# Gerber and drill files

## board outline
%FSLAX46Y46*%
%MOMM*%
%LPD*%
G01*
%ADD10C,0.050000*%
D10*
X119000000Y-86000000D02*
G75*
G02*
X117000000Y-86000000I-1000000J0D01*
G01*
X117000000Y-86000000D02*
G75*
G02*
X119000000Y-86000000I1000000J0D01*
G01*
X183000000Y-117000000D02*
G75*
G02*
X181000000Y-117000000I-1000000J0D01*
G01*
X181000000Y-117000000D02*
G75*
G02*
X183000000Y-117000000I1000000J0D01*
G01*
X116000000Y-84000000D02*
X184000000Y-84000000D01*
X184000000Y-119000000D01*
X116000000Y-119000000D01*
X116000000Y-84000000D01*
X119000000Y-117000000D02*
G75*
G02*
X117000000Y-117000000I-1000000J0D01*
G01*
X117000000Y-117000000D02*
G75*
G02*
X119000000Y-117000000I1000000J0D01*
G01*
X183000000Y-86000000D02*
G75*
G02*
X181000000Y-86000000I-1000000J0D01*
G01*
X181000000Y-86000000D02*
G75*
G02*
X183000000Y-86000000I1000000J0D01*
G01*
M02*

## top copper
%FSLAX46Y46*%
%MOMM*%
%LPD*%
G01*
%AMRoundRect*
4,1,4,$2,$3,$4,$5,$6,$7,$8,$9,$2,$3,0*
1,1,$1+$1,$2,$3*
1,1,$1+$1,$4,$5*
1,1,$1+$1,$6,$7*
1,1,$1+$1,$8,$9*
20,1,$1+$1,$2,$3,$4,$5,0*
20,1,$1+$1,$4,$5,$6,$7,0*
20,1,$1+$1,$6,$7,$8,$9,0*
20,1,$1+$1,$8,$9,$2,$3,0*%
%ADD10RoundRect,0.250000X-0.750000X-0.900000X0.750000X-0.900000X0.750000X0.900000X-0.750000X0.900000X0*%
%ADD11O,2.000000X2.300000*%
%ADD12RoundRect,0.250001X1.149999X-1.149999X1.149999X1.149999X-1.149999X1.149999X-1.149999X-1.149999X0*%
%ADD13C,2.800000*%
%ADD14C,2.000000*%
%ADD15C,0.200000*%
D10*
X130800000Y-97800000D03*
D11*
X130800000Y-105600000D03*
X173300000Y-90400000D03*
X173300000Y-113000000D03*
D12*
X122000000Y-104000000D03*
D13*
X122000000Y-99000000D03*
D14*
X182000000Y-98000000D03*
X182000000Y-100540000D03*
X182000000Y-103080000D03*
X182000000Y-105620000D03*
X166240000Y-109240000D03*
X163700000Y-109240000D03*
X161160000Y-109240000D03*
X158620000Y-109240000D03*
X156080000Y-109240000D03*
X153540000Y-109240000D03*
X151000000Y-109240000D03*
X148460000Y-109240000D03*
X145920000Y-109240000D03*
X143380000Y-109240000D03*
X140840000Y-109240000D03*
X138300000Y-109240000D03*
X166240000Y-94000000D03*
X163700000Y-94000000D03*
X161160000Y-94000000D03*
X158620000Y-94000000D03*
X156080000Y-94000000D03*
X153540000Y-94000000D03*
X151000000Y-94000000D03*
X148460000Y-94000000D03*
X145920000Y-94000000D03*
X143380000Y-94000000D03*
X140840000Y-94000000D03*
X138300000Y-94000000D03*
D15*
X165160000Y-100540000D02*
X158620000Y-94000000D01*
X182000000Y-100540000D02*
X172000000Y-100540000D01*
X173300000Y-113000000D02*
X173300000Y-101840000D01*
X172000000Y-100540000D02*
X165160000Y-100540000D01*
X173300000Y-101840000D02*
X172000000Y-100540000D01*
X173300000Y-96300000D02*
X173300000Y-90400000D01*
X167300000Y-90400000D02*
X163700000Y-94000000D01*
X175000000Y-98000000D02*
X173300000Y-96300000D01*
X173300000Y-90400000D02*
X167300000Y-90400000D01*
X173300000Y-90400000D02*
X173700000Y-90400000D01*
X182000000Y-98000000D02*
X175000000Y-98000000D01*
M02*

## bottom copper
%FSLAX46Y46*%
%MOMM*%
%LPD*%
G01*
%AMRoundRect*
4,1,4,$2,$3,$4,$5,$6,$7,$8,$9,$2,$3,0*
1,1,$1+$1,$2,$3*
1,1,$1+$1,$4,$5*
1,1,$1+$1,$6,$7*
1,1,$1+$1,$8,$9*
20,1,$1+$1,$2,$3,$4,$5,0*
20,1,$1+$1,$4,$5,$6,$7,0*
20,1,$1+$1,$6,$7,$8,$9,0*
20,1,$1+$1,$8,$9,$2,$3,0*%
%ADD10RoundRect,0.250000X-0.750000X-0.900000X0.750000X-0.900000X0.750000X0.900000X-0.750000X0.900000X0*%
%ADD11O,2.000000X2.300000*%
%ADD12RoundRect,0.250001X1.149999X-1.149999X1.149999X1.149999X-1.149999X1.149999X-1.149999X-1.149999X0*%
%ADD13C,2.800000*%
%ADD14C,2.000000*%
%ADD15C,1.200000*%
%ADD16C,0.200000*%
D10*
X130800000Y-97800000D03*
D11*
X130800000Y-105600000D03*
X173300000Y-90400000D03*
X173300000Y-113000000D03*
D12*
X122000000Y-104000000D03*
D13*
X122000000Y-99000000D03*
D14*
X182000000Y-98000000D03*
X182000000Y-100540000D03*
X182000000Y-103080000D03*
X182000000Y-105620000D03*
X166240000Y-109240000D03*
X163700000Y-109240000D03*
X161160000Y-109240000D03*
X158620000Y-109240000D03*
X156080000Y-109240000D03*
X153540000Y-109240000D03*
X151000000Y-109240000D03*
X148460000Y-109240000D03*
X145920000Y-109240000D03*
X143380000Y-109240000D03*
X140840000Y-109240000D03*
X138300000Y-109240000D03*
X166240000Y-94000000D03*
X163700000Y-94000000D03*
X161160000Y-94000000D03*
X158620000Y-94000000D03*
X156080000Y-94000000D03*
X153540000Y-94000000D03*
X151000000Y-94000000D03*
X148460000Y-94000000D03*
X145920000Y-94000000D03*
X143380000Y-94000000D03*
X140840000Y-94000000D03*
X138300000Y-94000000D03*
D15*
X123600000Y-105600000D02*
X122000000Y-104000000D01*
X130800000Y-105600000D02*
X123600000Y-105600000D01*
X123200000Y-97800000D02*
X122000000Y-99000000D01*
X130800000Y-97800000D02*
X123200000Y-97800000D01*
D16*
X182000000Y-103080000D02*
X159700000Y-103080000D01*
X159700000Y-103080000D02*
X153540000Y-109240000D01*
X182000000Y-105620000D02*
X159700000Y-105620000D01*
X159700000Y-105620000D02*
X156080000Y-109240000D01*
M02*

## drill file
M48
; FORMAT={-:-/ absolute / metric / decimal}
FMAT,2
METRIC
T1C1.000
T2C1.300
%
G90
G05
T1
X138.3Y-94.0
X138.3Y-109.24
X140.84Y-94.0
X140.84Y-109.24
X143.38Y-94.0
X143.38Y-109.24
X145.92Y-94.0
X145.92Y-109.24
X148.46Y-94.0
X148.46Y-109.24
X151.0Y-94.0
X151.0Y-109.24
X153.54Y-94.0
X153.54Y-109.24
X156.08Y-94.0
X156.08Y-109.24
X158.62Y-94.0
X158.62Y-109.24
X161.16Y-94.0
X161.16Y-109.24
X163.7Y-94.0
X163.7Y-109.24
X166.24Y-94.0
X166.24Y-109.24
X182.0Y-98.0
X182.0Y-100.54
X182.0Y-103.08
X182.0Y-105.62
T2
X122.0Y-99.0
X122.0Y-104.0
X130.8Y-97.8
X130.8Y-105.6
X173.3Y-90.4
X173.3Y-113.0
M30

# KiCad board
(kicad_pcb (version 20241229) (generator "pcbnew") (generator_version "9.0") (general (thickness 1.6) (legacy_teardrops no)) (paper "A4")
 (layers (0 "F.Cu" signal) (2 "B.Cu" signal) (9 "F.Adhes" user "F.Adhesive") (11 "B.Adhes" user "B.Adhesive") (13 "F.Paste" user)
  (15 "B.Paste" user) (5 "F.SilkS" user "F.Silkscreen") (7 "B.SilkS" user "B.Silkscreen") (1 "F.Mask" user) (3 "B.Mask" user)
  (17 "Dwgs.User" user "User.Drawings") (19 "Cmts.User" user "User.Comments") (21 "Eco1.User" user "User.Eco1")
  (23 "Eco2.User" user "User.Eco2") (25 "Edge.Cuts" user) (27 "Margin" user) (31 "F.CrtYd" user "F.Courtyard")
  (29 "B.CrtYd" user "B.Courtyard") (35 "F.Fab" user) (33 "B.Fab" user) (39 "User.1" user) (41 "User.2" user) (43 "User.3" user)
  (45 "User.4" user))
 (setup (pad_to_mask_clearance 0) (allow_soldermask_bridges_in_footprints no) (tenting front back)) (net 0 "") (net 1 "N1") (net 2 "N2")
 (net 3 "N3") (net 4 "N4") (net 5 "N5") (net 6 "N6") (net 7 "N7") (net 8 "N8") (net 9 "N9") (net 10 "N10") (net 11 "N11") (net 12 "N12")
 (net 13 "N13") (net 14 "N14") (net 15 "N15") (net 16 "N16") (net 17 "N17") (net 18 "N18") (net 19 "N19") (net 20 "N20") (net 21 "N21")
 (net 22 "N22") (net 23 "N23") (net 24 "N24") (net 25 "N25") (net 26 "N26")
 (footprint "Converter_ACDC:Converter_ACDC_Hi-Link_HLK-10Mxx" (layer "F.Cu") (at 130.8 97.8)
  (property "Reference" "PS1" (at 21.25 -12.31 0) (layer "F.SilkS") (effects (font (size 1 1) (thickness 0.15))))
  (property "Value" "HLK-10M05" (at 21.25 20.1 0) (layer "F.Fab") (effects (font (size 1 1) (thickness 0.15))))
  (pad "1" thru_hole roundrect (at 0 0) (size 2 2.3) (drill 1.3) (layers "*.Cu" "*.Mask") (remove_unused_layers no) (roundrect_rratio 0.125)
   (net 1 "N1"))
  (pad "2" thru_hole oval (at 0 7.8) (size 2 2.3) (drill 1.3) (layers "*.Cu" "*.Mask") (remove_unused_layers no) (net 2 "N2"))
  (pad "3" thru_hole oval (at 42.5 -7.4) (size 2 2.3) (drill 1.3) (layers "*.Cu" "*.Mask") (remove_unused_layers no) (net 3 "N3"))
  (pad "4" thru_hole oval (at 42.5 15.2) (size 2 2.3) (drill 1.3) (layers "*.Cu" "*.Mask") (remove_unused_layers no) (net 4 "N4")))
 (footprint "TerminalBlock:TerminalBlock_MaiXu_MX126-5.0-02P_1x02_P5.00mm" (layer "F.Cu") (at 122 104 90)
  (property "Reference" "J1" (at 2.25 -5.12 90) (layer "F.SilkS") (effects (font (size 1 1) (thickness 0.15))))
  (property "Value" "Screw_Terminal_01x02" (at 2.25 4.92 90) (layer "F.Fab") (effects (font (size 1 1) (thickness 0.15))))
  (pad "1" thru_hole roundrect (at 0 0 90) (size 2.8 2.8) (drill 1.3) (layers "*.Cu" "*.Mask") (remove_unused_layers no)
   (roundrect_rratio 0.089286) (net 2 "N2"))
  (pad "2" thru_hole circle (at 5 0 90) (size 2.8 2.8) (drill 1.3) (layers "*.Cu" "*.Mask") (remove_unused_layers no) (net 1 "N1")))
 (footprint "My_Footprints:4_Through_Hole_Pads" (layer "F.Cu") (at 174.38 103.08 -90)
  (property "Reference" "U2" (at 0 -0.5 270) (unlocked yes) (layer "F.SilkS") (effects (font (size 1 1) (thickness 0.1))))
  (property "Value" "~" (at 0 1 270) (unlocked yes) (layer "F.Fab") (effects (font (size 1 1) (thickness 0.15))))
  (pad "1" thru_hole circle (at -5.08 -7.62 270) (size 2 2) (drill 1) (layers "*.Cu" "*.Mask") (remove_unused_layers no) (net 3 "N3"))
  (pad "2" thru_hole circle (at -2.54 -7.62 270) (size 2 2) (drill 1) (layers "*.Cu" "*.Mask") (remove_unused_layers no) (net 4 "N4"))
  (pad "3" thru_hole circle (at 0 -7.62 270) (size 2 2) (drill 1) (layers "*.Cu" "*.Mask") (remove_unused_layers no) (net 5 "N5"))
  (pad "4" thru_hole circle (at 2.54 -7.62 270) (size 2 2) (drill 1) (layers "*.Cu" "*.Mask") (remove_unused_layers no) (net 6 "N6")))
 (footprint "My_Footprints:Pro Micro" (layer "B.Cu") (at 135.76 101.62 90)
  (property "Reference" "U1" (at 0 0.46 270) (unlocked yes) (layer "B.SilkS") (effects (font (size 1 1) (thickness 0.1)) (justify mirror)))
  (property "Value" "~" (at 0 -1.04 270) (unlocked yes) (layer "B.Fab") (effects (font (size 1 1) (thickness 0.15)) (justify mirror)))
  (pad "1" thru_hole circle (at -7.62 30.48 90) (size 2 2) (drill 1) (layers "*.Cu" "*.Mask") (remove_unused_layers no) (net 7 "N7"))
  (pad "2" thru_hole circle (at -7.62 27.94 90) (size 2 2) (drill 1) (layers "*.Cu" "*.Mask") (remove_unused_layers no) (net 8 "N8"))
  (pad "3" thru_hole circle (at -7.62 25.4 90) (size 2 2) (drill 1) (layers "*.Cu" "*.Mask") (remove_unused_layers no) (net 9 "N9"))
  (pad "4" thru_hole circle (at -7.62 22.86 90) (size 2 2) (drill 1) (layers "*.Cu" "*.Mask") (remove_unused_layers no) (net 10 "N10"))
  (pad "5" thru_hole circle (at -7.62 20.32 90) (size 2 2) (drill 1) (layers "*.Cu" "*.Mask") (remove_unused_layers no) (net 6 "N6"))
  (pad "6" thru_hole circle (at -7.62 17.78 90) (size 2 2) (drill 1) (layers "*.Cu" "*.Mask") (remove_unused_layers no) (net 5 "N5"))
  (pad "7" thru_hole circle (at -7.62 15.24 90) (size 2 2) (drill 1) (layers "*.Cu" "*.Mask") (remove_unused_layers no) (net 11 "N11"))
  (pad "8" thru_hole circle (at -7.62 12.7 90) (size 2 2) (drill 1) (layers "*.Cu" "*.Mask") (remove_unused_layers no) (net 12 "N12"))
  (pad "9" thru_hole circle (at -7.62 10.16 90) (size 2 2) (drill 1) (layers "*.Cu" "*.Mask") (remove_unused_layers no) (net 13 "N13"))
  (pad "10" thru_hole circle (at -7.62 7.62 180) (size 2 2) (drill 1) (layers "*.Cu" "*.Mask") (remove_unused_layers no) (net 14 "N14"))
  (pad "11" thru_hole circle (at -7.62 5.08 90) (size 2 2) (drill 1) (layers "*.Cu" "*.Mask") (remove_unused_layers no) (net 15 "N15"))
  (pad "12" thru_hole circle (at -7.62 2.54 90) (size 2 2) (drill 1) (layers "*.Cu" "*.Mask") (remove_unused_layers no) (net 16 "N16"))
  (pad "13" thru_hole circle (at 7.62 30.48 90) (size 2 2) (drill 1) (layers "*.Cu" "*.Mask") (remove_unused_layers no) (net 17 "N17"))
  (pad "14" thru_hole circle (at 7.62 27.94 90) (size 2 2) (drill 1) (layers "*.Cu" "*.Mask") (remove_unused_layers no) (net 3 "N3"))
  (pad "15" thru_hole circle (at 7.62 25.4 270) (size 2 2) (drill 1) (layers "*.Cu" "*.Mask") (remove_unused_layers no) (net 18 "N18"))
  (pad "16" thru_hole circle (at 7.62 22.86) (size 2 2) (drill 1) (layers "*.Cu" "*.Mask") (remove_unused_layers no) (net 4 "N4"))
  (pad "17" thru_hole circle (at 7.62 20.32 90) (size 2 2) (drill 1) (layers "*.Cu" "*.Mask") (remove_unused_layers no) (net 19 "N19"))
  (pad "18" thru_hole circle (at 7.62 17.78 90) (size 2 2) (drill 1) (layers "*.Cu" "*.Mask") (remove_unused_layers no) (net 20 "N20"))
  (pad "19" thru_hole circle (at 7.62 15.24 90) (size 2 2) (drill 1) (layers "*.Cu" "*.Mask") (remove_unused_layers no) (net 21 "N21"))
  (pad "20" thru_hole circle (at 7.62 12.7 90) (size 2 2) (drill 1) (layers "*.Cu" "*.Mask") (remove_unused_layers no) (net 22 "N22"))
  (pad "21" thru_hole circle (at 7.62 10.16 90) (size 2 2) (drill 1) (layers "*.Cu" "*.Mask") (remove_unused_layers no) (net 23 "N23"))
  (pad "22" thru_hole circle (at 7.62 7.62 90) (size 2 2) (drill 1) (layers "*.Cu" "*.Mask") (remove_unused_layers no) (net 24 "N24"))
  (pad "23" thru_hole circle (at 7.62 5.08 90) (size 2 2) (drill 1) (layers "*.Cu" "*.Mask") (remove_unused_layers no) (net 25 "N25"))
  (pad "24" thru_hole circle (at 7.62 2.54 90) (size 2 2) (drill 1) (layers "*.Cu" "*.Mask") (remove_unused_layers no) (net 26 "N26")))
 (gr_circle (center 118 86) (end 119 86) (stroke (width 0.05) (type default)) (fill no) (layer "Edge.Cuts"))
 (gr_circle (center 182 117) (end 182 118) (stroke (width 0.05) (type default)) (fill no) (layer "Edge.Cuts"))
 (gr_rect (start 116 84) (end 184 119) (stroke (width 0.05) (type default)) (fill no) (layer "Edge.Cuts"))
 (gr_circle (center 118 117) (end 119 117) (stroke (width 0.05) (type default)) (fill no) (layer "Edge.Cuts"))
 (gr_circle (center 182 86) (end 183 86) (stroke (width 0.05) (type default)) (fill no) (layer "Edge.Cuts"))
 (segment (start 123.6 105.6) (end 122 104) (width 1.2) (layer "B.Cu") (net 2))
 (segment (start 130.8 105.6) (end 123.6 105.6) (width 1.2) (layer "B.Cu") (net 2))
 (segment (start 123.2 97.8) (end 122 99) (width 1.2) (layer "B.Cu") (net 1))
 (segment (start 130.8 97.8) (end 123.2 97.8) (width 1.2) (layer "B.Cu") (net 1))
 (segment (start 165.16 100.54) (end 158.62 94) (width 0.2) (layer "F.Cu") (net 4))
 (segment (start 182 100.54) (end 172 100.54) (width 0.2) (layer "F.Cu") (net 4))
 (segment (start 173.3 113) (end 173.3 101.84) (width 0.2) (layer "F.Cu") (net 4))
 (segment (start 172 100.54) (end 165.16 100.54) (width 0.2) (layer "F.Cu") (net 4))
 (segment (start 173.3 101.84) (end 172 100.54) (width 0.2) (layer "F.Cu") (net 4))
 (segment (start 173.3 96.3) (end 173.3 90.4) (width 0.2) (layer "F.Cu") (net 3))
 (segment (start 167.3 90.4) (end 163.7 94) (width 0.2) (layer "F.Cu") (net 3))
 (segment (start 175 98) (end 173.3 96.3) (width 0.2) (layer "F.Cu") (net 3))
 (segment (start 173.3 90.4) (end 167.3 90.4) (width 0.2) (layer "F.Cu") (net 3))
 (segment (start 173.3 90.4) (end 173.7 90.4) (width 0.2) (layer "F.Cu") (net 3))
 (segment (start 182 98) (end 175 98) (width 0.2) (layer "F.Cu") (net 3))
 (segment (start 182 103.08) (end 159.7 103.08) (width 0.2) (layer "B.Cu") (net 5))
 (segment (start 159.7 103.08) (end 153.54 109.24) (width 0.2) (layer "B.Cu") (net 5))
 (segment (start 182 105.62) (end 159.7 105.62) (width 0.2) (layer "B.Cu") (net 6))
 (segment (start 159.7 105.62) (end 156.08 109.24) (width 0.2) (layer "B.Cu") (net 6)))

